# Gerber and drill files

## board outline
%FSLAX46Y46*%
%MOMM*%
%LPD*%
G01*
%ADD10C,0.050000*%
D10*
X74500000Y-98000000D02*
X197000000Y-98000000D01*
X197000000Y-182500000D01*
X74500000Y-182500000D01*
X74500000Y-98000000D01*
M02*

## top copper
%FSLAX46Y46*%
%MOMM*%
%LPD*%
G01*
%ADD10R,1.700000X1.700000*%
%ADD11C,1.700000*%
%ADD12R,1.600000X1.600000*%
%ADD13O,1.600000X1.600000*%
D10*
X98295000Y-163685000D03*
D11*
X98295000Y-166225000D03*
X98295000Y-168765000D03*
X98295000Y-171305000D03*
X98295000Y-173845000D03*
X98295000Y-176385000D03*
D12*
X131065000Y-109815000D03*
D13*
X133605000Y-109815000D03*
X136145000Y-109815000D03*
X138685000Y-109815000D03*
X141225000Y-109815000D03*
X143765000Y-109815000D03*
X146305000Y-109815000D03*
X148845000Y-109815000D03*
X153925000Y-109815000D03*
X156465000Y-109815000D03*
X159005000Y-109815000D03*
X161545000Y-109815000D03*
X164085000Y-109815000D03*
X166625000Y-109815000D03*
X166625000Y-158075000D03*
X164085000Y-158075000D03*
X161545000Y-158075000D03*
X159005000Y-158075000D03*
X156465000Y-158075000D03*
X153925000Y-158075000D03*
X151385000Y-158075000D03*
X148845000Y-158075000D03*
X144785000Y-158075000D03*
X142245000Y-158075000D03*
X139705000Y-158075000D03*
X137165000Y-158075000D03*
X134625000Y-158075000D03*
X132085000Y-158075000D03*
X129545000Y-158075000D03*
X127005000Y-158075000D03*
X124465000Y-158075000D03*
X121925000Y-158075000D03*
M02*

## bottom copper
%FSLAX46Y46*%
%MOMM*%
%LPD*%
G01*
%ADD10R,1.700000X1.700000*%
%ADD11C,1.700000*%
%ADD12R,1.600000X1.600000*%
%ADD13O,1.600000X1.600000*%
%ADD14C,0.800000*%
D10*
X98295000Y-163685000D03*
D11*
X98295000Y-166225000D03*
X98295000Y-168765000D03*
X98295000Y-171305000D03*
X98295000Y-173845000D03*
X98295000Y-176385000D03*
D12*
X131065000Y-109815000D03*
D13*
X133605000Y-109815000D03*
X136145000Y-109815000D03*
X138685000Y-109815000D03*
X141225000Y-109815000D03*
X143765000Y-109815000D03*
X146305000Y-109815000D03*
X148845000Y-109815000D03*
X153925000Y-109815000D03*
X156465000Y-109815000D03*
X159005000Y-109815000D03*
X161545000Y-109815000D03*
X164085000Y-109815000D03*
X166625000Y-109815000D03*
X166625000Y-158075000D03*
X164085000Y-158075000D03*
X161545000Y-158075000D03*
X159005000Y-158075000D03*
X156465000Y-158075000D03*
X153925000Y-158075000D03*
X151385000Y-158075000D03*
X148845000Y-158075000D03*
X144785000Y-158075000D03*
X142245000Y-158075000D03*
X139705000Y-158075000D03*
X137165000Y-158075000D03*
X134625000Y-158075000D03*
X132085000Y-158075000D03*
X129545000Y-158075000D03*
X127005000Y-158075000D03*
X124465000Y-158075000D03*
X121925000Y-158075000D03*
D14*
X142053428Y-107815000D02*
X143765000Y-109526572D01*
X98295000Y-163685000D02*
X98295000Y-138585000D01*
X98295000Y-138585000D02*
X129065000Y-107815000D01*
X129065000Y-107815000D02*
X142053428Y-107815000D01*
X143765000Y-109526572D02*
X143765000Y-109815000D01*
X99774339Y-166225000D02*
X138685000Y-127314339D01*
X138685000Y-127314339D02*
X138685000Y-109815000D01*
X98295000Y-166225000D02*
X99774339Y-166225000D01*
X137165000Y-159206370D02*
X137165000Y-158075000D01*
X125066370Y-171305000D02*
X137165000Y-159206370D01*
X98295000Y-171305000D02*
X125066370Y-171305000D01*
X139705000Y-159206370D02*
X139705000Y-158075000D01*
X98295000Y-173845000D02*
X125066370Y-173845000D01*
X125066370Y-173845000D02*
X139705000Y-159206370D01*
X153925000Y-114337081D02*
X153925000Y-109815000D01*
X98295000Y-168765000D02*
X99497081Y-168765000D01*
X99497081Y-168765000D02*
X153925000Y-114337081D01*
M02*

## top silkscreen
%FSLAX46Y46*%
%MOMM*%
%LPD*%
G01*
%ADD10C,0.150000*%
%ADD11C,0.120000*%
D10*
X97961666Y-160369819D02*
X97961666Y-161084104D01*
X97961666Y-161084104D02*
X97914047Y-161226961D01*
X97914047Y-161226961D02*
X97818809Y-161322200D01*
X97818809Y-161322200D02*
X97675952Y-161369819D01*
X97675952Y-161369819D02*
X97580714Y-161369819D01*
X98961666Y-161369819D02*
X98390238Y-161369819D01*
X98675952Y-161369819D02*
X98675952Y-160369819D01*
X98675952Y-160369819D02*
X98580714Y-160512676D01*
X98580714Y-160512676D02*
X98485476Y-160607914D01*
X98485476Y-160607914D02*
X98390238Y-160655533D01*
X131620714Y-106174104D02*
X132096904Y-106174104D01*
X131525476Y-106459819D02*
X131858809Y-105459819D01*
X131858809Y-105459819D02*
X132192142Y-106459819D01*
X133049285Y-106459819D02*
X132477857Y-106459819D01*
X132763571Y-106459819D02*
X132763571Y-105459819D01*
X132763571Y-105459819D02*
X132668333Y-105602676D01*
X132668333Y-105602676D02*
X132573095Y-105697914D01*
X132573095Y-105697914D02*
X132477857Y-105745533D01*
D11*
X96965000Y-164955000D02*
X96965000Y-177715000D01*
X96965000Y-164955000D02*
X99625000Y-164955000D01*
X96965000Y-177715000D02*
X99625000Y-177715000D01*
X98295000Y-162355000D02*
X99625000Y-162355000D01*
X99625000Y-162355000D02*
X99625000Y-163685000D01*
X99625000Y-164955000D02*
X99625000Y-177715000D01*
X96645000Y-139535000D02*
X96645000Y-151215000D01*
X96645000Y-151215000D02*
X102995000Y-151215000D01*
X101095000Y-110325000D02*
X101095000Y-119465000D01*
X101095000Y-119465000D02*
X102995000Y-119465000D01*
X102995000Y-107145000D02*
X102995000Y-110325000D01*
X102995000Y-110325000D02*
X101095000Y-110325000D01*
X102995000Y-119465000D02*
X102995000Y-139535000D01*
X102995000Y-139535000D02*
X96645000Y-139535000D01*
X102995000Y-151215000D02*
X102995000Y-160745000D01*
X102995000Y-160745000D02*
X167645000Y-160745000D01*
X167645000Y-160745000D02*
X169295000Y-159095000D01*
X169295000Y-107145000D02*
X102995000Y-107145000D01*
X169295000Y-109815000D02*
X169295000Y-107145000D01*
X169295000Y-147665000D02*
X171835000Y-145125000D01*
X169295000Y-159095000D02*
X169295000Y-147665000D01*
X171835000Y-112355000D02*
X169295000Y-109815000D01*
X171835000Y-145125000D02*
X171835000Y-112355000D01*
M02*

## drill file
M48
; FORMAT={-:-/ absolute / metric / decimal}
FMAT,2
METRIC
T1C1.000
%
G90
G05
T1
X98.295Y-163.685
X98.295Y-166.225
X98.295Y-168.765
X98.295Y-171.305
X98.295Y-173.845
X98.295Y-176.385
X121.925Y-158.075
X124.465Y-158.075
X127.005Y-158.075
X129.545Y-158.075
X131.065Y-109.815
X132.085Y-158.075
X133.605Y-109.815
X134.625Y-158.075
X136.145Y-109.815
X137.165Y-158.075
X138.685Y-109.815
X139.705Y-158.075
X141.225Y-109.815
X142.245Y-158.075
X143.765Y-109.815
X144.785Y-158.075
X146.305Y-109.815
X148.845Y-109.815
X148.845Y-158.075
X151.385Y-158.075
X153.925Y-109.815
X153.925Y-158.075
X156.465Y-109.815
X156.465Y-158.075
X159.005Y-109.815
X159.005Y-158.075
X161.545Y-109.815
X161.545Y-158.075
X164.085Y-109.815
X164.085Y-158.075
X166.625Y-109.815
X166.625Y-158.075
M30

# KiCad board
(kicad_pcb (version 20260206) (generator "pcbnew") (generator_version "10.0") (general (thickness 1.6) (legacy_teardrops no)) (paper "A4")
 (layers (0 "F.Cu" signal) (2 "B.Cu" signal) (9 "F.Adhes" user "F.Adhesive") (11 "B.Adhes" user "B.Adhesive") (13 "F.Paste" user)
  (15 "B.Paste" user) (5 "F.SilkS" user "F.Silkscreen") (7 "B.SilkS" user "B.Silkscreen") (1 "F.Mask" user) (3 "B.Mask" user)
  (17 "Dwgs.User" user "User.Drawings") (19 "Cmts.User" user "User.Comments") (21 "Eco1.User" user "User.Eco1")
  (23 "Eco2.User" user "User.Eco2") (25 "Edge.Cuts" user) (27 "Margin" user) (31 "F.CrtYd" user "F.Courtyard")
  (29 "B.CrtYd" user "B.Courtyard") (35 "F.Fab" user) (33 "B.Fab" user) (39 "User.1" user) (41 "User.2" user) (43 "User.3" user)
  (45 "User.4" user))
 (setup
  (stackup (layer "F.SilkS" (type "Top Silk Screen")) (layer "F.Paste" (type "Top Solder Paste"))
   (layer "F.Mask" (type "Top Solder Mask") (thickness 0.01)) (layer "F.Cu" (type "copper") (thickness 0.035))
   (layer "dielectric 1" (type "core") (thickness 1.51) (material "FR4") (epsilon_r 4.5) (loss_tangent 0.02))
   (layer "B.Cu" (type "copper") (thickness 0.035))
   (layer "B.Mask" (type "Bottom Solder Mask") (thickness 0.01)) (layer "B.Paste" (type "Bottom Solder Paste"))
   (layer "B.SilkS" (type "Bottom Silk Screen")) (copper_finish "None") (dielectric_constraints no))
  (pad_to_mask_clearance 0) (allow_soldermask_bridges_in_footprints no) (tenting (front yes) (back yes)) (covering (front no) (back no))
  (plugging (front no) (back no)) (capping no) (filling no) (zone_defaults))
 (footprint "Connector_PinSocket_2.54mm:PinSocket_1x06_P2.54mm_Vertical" (layer "F.Cu") (at 98.295 163.685)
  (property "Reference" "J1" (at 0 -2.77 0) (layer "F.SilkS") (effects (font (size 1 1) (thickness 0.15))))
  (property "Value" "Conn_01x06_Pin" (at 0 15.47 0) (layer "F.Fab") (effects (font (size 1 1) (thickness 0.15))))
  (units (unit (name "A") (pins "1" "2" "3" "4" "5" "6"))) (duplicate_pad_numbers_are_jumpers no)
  (fp_line (start -1.33 1.27) (end -1.33 14.03) (stroke (width 0.12) (type solid)) (layer "F.SilkS"))
  (fp_line (start -1.33 1.27) (end 1.33 1.27) (stroke (width 0.12) (type solid)) (layer "F.SilkS"))
  (fp_line (start -1.33 14.03) (end 1.33 14.03) (stroke (width 0.12) (type solid)) (layer "F.SilkS"))
  (fp_line (start 0 -1.33) (end 1.33 -1.33) (stroke (width 0.12) (type solid)) (layer "F.SilkS"))
  (fp_line (start 1.33 -1.33) (end 1.33 0) (stroke (width 0.12) (type solid)) (layer "F.SilkS"))
  (fp_line (start 1.33 1.27) (end 1.33 14.03) (stroke (width 0.12) (type solid)) (layer "F.SilkS"))
  (pad "1" thru_hole rect (at 0 0) (size 1.7 1.7) (drill 1) (layers "*.Cu" "*.Mask") (remove_unused_layers no) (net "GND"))
  (pad "2" thru_hole circle (at 0 2.54) (size 1.7 1.7) (drill 1) (layers "*.Cu" "*.Mask") (remove_unused_layers no) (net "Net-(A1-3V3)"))
  (pad "3" thru_hole circle (at 0 5.08) (size 1.7 1.7) (drill 1) (layers "*.Cu" "*.Mask") (remove_unused_layers no) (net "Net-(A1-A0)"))
  (pad "4" thru_hole circle (at 0 7.62) (size 1.7 1.7) (drill 1) (layers "*.Cu" "*.Mask") (remove_unused_layers no) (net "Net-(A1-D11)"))
  (pad "5" thru_hole circle (at 0 10.16) (size 1.7 1.7) (drill 1) (layers "*.Cu" "*.Mask") (remove_unused_layers no) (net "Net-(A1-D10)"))
  (pad "6" thru_hole circle (at 0 12.7) (size 1.7 1.7) (drill 1) (layers "*.Cu" "*.Mask") (remove_unused_layers no)
   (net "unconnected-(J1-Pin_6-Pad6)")))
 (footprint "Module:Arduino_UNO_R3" (layer "F.Cu") (at 131.065 109.815)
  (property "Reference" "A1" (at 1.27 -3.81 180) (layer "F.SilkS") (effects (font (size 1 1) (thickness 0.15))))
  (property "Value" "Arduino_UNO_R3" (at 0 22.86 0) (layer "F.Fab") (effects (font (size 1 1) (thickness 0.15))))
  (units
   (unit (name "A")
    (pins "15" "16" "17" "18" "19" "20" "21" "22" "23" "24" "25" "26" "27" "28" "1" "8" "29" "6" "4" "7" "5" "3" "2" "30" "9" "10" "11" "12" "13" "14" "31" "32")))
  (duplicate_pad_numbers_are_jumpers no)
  (fp_line (start -34.42 29.72) (end -34.42 41.4) (stroke (width 0.12) (type solid)) (layer "F.SilkS"))
  (fp_line (start -34.42 41.4) (end -28.07 41.4) (stroke (width 0.12) (type solid)) (layer "F.SilkS"))
  (fp_line (start -29.97 0.51) (end -29.97 9.65) (stroke (width 0.12) (type solid)) (layer "F.SilkS"))
  (fp_line (start -29.97 9.65) (end -28.07 9.65) (stroke (width 0.12) (type solid)) (layer "F.SilkS"))
  (fp_line (start -28.07 -2.67) (end -28.07 0.51) (stroke (width 0.12) (type solid)) (layer "F.SilkS"))
  (fp_line (start -28.07 0.51) (end -29.97 0.51) (stroke (width 0.12) (type solid)) (layer "F.SilkS"))
  (fp_line (start -28.07 9.65) (end -28.07 29.72) (stroke (width 0.12) (type solid)) (layer "F.SilkS"))
  (fp_line (start -28.07 29.72) (end -34.42 29.72) (stroke (width 0.12) (type solid)) (layer "F.SilkS"))
  (fp_line (start -28.07 41.4) (end -28.07 50.93) (stroke (width 0.12) (type solid)) (layer "F.SilkS"))
  (fp_line (start -28.07 50.93) (end 36.58 50.93) (stroke (width 0.12) (type solid)) (layer "F.SilkS"))
  (fp_line (start 36.58 50.93) (end 38.23 49.28) (stroke (width 0.12) (type solid)) (layer "F.SilkS"))
  (fp_line (start 38.23 -2.67) (end -28.07 -2.67) (stroke (width 0.12) (type solid)) (layer "F.SilkS"))
  (fp_line (start 38.23 0) (end 38.23 -2.67) (stroke (width 0.12) (type solid)) (layer "F.SilkS"))
  (fp_line (start 38.23 37.85) (end 40.77 35.31) (stroke (width 0.12) (type solid)) (layer "F.SilkS"))
  (fp_line (start 38.23 49.28) (end 38.23 37.85) (stroke (width 0.12) (type solid)) (layer "F.SilkS"))
  (fp_line (start 40.77 2.54) (end 38.23 0) (stroke (width 0.12) (type solid)) (layer "F.SilkS"))
  (fp_line (start 40.77 35.31) (end 40.77 2.54) (stroke (width 0.12) (type solid)) (layer "F.SilkS"))
  (pad "1" thru_hole rect (at 0 0 90) (size 1.6 1.6) (drill 1) (layers "*.Cu" "*.Mask") (remove_unused_layers no)
   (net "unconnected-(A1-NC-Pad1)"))
  (pad "2" thru_hole oval (at 2.54 0 90) (size 1.6 1.6) (drill 1) (layers "*.Cu" "*.Mask") (remove_unused_layers no)
   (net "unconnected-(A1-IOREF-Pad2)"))
  (pad "3" thru_hole oval (at 5.08 0 90) (size 1.6 1.6) (drill 1) (layers "*.Cu" "*.Mask") (remove_unused_layers no)
   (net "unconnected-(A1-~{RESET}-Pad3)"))
  (pad "4" thru_hole oval (at 7.62 0 90) (size 1.6 1.6) (drill 1) (layers "*.Cu" "*.Mask") (remove_unused_layers no) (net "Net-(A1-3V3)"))
  (pad "5" thru_hole oval (at 10.16 0 90) (size 1.6 1.6) (drill 1) (layers "*.Cu" "*.Mask") (remove_unused_layers no)
   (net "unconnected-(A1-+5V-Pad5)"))
  (pad "6" thru_hole oval (at 12.7 0 90) (size 1.6 1.6) (drill 1) (layers "*.Cu" "*.Mask") (remove_unused_layers no) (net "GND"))
  (pad "7" thru_hole oval (at 15.24 0 90) (size 1.6 1.6) (drill 1) (layers "*.Cu" "*.Mask") (remove_unused_layers no)
   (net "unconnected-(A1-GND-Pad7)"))
  (pad "8" thru_hole oval (at 17.78 0 90) (size 1.6 1.6) (drill 1) (layers "*.Cu" "*.Mask") (remove_unused_layers no)
   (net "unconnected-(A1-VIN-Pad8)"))
  (pad "9" thru_hole oval (at 22.86 0 90) (size 1.6 1.6) (drill 1) (layers "*.Cu" "*.Mask") (remove_unused_layers no) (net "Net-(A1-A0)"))
  (pad "10" thru_hole oval (at 25.4 0 90) (size 1.6 1.6) (drill 1) (layers "*.Cu" "*.Mask") (remove_unused_layers no)
   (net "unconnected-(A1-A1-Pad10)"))
  (pad "11" thru_hole oval (at 27.94 0 90) (size 1.6 1.6) (drill 1) (layers "*.Cu" "*.Mask") (remove_unused_layers no)
   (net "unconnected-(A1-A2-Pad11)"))
  (pad "12" thru_hole oval (at 30.48 0 90) (size 1.6 1.6) (drill 1) (layers "*.Cu" "*.Mask") (remove_unused_layers no)
   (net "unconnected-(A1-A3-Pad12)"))
  (pad "13" thru_hole oval (at 33.02 0 90) (size 1.6 1.6) (drill 1) (layers "*.Cu" "*.Mask") (remove_unused_layers no)
   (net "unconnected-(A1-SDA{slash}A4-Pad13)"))
  (pad "14" thru_hole oval (at 35.56 0 90) (size 1.6 1.6) (drill 1) (layers "*.Cu" "*.Mask") (remove_unused_layers no)
   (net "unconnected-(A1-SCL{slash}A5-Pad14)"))
  (pad "15" thru_hole oval (at 35.56 48.26 90) (size 1.6 1.6) (drill 1) (layers "*.Cu" "*.Mask") (remove_unused_layers no)
   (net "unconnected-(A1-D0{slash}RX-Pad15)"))
  (pad "16" thru_hole oval (at 33.02 48.26 90) (size 1.6 1.6) (drill 1) (layers "*.Cu" "*.Mask") (remove_unused_layers no)
   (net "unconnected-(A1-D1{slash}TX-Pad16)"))
  (pad "17" thru_hole oval (at 30.48 48.26 90) (size 1.6 1.6) (drill 1) (layers "*.Cu" "*.Mask") (remove_unused_layers no)
   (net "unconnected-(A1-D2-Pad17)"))
  (pad "18" thru_hole oval (at 27.94 48.26 90) (size 1.6 1.6) (drill 1) (layers "*.Cu" "*.Mask") (remove_unused_layers no)
   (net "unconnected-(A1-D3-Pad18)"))
  (pad "19" thru_hole oval (at 25.4 48.26 90) (size 1.6 1.6) (drill 1) (layers "*.Cu" "*.Mask") (remove_unused_layers no)
   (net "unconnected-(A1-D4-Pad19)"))
  (pad "20" thru_hole oval (at 22.86 48.26 90) (size 1.6 1.6) (drill 1) (layers "*.Cu" "*.Mask") (remove_unused_layers no)
   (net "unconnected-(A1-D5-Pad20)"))
  (pad "21" thru_hole oval (at 20.32 48.26 90) (size 1.6 1.6) (drill 1) (layers "*.Cu" "*.Mask") (remove_unused_layers no)
   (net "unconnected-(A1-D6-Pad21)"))
  (pad "22" thru_hole oval (at 17.78 48.26 90) (size 1.6 1.6) (drill 1) (layers "*.Cu" "*.Mask") (remove_unused_layers no)
   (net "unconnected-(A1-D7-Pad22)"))
  (pad "23" thru_hole oval (at 13.72 48.26 90) (size 1.6 1.6) (drill 1) (layers "*.Cu" "*.Mask") (remove_unused_layers no)
   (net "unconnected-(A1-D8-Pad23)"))
  (pad "24" thru_hole oval (at 11.18 48.26 90) (size 1.6 1.6) (drill 1) (layers "*.Cu" "*.Mask") (remove_unused_layers no)
   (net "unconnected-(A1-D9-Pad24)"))
  (pad "25" thru_hole oval (at 8.64 48.26 90) (size 1.6 1.6) (drill 1) (layers "*.Cu" "*.Mask") (remove_unused_layers no)
   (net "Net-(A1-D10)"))
  (pad "26" thru_hole oval (at 6.1 48.26 90) (size 1.6 1.6) (drill 1) (layers "*.Cu" "*.Mask") (remove_unused_layers no)
   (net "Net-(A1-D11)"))
  (pad "27" thru_hole oval (at 3.56 48.26 90) (size 1.6 1.6) (drill 1) (layers "*.Cu" "*.Mask") (remove_unused_layers no)
   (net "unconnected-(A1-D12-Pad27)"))
  (pad "28" thru_hole oval (at 1.02 48.26 90) (size 1.6 1.6) (drill 1) (layers "*.Cu" "*.Mask") (remove_unused_layers no)
   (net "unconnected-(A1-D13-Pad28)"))
  (pad "29" thru_hole oval (at -1.52 48.26 90) (size 1.6 1.6) (drill 1) (layers "*.Cu" "*.Mask") (remove_unused_layers no)
   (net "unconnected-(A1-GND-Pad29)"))
  (pad "30" thru_hole oval (at -4.06 48.26 90) (size 1.6 1.6) (drill 1) (layers "*.Cu" "*.Mask") (remove_unused_layers no)
   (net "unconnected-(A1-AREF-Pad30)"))
  (pad "31" thru_hole oval (at -6.6 48.26 90) (size 1.6 1.6) (drill 1) (layers "*.Cu" "*.Mask") (remove_unused_layers no)
   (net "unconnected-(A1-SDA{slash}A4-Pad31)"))
  (pad "32" thru_hole oval (at -9.14 48.26 90) (size 1.6 1.6) (drill 1) (layers "*.Cu" "*.Mask") (remove_unused_layers no)
   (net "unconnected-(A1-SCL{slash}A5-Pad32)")))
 (gr_rect (start 74.5 98) (end 197 182.5) (stroke (width 0.05) (type default)) (fill no) (layer "Edge.Cuts"))
 (segment (start 142.053428 107.815) (end 143.765 109.526572) (width 0.8) (layer "B.Cu") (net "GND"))
 (segment (start 98.295 163.685) (end 98.295 138.585) (width 0.8) (layer "B.Cu") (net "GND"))
 (segment (start 98.295 138.585) (end 129.065 107.815) (width 0.8) (layer "B.Cu") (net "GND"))
 (segment (start 129.065 107.815) (end 142.053428 107.815) (width 0.8) (layer "B.Cu") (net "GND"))
 (segment (start 143.765 109.526572) (end 143.765 109.815) (width 0.8) (layer "B.Cu") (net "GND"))
 (segment (start 99.774339 166.225) (end 138.685 127.314339) (width 0.8) (layer "B.Cu") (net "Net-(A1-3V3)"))
 (segment (start 138.685 127.314339) (end 138.685 109.815) (width 0.8) (layer "B.Cu") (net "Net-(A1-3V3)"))
 (segment (start 98.295 166.225) (end 99.774339 166.225) (width 0.8) (layer "B.Cu") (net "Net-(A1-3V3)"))
 (segment (start 137.165 159.20637) (end 137.165 158.075) (width 0.8) (layer "B.Cu") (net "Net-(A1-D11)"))
 (segment (start 125.06637 171.305) (end 137.165 159.20637) (width 0.8) (layer "B.Cu") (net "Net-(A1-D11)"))
 (segment (start 98.295 171.305) (end 125.06637 171.305) (width 0.8) (layer "B.Cu") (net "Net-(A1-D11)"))
 (segment (start 139.705 159.20637) (end 139.705 158.075) (width 0.8) (layer "B.Cu") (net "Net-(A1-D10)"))
 (segment (start 98.295 173.845) (end 125.06637 173.845) (width 0.8) (layer "B.Cu") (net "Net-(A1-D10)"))
 (segment (start 125.06637 173.845) (end 139.705 159.20637) (width 0.8) (layer "B.Cu") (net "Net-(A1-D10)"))
 (segment (start 153.925 114.337081) (end 153.925 109.815) (width 0.8) (layer "B.Cu") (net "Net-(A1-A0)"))
 (segment (start 98.295 168.765) (end 99.497081 168.765) (width 0.8) (layer "B.Cu") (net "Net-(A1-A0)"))
 (segment (start 99.497081 168.765) (end 153.925 114.337081) (width 0.8) (layer "B.Cu") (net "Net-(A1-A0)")))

